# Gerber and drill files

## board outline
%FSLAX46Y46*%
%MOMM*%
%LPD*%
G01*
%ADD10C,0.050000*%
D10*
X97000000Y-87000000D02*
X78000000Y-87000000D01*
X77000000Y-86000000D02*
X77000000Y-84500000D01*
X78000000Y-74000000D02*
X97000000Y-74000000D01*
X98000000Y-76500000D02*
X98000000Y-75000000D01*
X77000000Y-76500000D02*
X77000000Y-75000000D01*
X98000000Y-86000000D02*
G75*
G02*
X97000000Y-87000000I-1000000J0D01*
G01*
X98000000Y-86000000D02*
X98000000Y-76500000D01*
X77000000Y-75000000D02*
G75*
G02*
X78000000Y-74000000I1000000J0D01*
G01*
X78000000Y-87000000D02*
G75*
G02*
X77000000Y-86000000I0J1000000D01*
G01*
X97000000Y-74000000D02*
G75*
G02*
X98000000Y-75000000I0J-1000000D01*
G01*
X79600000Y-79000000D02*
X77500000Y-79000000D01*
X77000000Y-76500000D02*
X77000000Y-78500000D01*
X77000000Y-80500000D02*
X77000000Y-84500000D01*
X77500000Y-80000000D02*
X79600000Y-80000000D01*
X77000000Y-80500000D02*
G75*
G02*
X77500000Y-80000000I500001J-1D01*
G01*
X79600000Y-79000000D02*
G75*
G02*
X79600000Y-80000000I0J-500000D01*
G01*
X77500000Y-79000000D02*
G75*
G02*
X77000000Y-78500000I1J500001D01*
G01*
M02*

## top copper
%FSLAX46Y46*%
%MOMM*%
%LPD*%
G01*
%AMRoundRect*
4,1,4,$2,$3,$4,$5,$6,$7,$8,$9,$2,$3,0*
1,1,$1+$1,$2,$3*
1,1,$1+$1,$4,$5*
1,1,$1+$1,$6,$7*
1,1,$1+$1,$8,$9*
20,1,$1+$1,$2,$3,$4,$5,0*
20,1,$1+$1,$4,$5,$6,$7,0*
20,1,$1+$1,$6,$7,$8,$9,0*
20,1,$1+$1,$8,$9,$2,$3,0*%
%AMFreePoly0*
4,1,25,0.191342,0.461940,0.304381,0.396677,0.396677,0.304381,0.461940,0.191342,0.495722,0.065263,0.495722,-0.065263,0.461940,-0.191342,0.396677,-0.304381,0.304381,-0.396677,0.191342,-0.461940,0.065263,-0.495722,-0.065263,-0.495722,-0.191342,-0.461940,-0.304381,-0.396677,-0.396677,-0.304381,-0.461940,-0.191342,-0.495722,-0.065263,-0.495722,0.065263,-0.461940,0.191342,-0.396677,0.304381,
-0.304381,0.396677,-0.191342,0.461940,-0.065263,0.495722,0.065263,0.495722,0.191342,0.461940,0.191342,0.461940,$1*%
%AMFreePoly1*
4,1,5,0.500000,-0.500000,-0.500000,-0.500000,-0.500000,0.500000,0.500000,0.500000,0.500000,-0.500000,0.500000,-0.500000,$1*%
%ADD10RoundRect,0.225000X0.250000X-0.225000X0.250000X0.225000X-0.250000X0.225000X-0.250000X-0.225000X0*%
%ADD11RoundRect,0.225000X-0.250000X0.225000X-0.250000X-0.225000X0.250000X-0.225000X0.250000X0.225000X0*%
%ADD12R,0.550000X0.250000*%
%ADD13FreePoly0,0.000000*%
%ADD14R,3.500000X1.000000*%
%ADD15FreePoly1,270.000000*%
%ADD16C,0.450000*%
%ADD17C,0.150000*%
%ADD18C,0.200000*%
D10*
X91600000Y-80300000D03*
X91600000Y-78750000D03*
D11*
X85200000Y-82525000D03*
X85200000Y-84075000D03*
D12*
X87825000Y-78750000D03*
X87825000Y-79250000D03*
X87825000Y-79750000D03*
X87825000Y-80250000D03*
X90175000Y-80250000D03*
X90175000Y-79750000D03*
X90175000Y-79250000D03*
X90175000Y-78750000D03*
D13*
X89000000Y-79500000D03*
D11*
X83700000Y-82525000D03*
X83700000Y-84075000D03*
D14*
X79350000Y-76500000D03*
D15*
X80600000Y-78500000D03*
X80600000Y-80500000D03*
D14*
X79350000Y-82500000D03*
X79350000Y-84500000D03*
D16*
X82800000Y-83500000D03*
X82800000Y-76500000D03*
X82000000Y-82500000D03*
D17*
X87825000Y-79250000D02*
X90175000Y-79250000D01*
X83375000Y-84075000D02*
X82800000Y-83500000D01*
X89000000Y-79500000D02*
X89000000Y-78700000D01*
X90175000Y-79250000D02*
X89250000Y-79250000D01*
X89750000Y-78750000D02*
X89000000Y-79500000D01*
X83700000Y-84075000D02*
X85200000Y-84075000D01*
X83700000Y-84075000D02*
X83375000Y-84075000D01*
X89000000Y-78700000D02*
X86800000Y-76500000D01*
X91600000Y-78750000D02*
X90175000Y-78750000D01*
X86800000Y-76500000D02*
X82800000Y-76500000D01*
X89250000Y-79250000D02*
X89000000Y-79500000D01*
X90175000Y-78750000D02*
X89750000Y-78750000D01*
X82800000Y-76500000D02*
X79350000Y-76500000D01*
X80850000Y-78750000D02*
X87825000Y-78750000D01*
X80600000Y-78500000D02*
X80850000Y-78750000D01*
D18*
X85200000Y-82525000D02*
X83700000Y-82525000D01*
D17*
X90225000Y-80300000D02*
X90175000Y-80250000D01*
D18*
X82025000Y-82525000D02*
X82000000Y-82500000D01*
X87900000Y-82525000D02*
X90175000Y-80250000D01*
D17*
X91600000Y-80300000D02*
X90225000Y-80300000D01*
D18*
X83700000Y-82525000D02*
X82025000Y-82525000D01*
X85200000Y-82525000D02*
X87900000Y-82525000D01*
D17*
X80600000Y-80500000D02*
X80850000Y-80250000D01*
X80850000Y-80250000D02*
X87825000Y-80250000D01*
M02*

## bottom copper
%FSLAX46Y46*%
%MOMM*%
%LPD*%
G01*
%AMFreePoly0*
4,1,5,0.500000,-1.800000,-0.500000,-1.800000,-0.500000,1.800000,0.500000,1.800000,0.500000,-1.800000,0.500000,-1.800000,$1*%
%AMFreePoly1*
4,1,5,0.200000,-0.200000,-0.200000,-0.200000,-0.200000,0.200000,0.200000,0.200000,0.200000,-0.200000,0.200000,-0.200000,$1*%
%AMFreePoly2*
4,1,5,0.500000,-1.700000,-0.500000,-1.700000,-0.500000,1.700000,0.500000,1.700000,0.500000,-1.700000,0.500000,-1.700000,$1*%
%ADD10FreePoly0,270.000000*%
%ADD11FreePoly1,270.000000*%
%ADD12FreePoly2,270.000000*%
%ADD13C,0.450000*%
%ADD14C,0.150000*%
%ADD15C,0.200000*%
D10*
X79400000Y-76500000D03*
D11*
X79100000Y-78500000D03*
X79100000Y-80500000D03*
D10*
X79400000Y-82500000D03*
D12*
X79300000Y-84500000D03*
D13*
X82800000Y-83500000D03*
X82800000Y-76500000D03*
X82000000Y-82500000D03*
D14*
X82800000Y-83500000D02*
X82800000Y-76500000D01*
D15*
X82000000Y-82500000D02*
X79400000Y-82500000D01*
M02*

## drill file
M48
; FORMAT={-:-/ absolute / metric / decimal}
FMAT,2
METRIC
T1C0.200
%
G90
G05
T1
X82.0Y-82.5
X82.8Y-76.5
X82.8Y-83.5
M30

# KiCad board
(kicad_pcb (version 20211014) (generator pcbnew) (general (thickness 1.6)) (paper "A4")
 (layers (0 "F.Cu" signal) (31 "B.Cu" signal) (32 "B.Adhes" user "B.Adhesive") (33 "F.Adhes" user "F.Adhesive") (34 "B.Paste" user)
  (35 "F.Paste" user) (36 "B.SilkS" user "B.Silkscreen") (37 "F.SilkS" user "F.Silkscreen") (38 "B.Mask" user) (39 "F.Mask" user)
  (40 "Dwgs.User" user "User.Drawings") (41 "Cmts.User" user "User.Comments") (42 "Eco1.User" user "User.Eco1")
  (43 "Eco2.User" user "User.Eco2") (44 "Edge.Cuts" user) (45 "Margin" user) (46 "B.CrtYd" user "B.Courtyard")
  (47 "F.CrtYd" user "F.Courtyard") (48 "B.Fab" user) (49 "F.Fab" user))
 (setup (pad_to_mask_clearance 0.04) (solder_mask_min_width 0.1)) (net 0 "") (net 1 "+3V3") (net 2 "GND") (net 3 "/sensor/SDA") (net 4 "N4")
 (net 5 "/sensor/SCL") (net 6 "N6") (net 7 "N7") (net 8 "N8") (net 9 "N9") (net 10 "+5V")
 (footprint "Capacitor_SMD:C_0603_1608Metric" (layer "F.Cu") (at 91.6 79.525 90)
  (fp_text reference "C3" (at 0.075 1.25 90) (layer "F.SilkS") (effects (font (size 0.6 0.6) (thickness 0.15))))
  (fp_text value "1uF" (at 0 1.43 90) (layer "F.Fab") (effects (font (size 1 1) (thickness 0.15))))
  (pad "1" smd roundrect locked (at -0.775 0 90) (size 0.9 0.95) (layers "F.Cu" "F.Paste" "F.Mask") (roundrect_rratio 0.25) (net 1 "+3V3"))
  (pad "2" smd roundrect locked (at 0.775 0 90) (size 0.9 0.95) (layers "F.Cu" "F.Paste" "F.Mask") (roundrect_rratio 0.25) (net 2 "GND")))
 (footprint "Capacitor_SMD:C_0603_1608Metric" (layer "F.Cu") (at 85.2 83.3 -90)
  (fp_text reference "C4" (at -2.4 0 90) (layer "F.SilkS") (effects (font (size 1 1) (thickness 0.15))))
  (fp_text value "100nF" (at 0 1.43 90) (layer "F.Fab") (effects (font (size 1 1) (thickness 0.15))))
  (pad "1" smd roundrect locked (at -0.775 0 270) (size 0.9 0.95) (layers "F.Cu" "F.Paste" "F.Mask") (roundrect_rratio 0.25) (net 1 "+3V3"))
  (pad "2" smd roundrect locked (at 0.775 0 270) (size 0.9 0.95) (layers "F.Cu" "F.Paste" "F.Mask") (roundrect_rratio 0.25) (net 2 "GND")))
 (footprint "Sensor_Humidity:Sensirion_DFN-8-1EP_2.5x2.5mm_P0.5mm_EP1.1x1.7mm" (layer "F.Cu") (at 89 79.5)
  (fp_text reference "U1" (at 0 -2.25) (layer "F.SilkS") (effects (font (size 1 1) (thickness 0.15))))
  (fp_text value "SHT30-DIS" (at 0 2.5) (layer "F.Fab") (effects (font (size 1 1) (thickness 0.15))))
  (pad "" smd custom (at 0 0) (size 0.9 0.9) (layers "F.Paste") (zone_connect 0) (options (clearance outline) (anchor rect)) (primitives))
  (pad "1" smd rect (at -1.175 -0.75) (size 0.55 0.25) (layers "F.Cu" "F.Paste" "F.Mask") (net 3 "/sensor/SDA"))
  (pad "2" smd rect (at -1.175 -0.25) (size 0.55 0.25) (layers "F.Cu" "F.Paste" "F.Mask") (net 2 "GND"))
  (pad "3" smd rect (at -1.175 0.25) (size 0.55 0.25) (layers "F.Cu" "F.Paste" "F.Mask") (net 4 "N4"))
  (pad "4" smd rect (at -1.175 0.75 180) (size 0.55 0.25) (layers "F.Cu" "F.Paste" "F.Mask") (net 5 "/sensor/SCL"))
  (pad "5" smd rect (at 1.175 0.75) (size 0.55 0.25) (layers "F.Cu" "F.Paste" "F.Mask") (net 1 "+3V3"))
  (pad "6" smd rect (at 1.175 0.25) (size 0.55 0.25) (layers "F.Cu" "F.Paste" "F.Mask") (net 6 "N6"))
  (pad "7" smd rect (at 1.175 -0.25) (size 0.55 0.25) (layers "F.Cu" "F.Paste" "F.Mask") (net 2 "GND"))
  (pad "8" smd rect (at 1.175 -0.75) (size 0.55 0.25) (layers "F.Cu" "F.Paste" "F.Mask") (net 2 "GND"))
  (pad "9" smd custom (at 0 0) (size 1 1) (layers "F.Cu" "F.Mask") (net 2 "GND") (zone_connect 0)
   (options (clearance outline) (anchor circle)) (primitives)))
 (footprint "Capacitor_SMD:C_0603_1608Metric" (layer "F.Cu") (at 83.7 83.3 -90)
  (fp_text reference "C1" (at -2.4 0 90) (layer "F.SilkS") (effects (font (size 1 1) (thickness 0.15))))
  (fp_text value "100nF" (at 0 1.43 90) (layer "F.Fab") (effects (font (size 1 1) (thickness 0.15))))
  (pad "1" smd roundrect (at -0.775 0 270) (size 0.9 0.95) (layers "F.Cu" "F.Paste" "F.Mask") (roundrect_rratio 0.25) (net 1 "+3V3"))
  (pad "2" smd roundrect (at 0.775 0 270) (size 0.9 0.95) (layers "F.Cu" "F.Paste" "F.Mask") (roundrect_rratio 0.25) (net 2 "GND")))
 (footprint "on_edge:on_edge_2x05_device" (layer "F.Cu") (at 77 80.5 -90)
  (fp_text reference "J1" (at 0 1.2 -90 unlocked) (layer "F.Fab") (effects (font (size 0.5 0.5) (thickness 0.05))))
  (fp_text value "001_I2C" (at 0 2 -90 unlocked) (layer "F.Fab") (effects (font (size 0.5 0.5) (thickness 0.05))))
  (fp_line (start -1.5 -2.6) (end -1.5 -0.5) (layer "Edge.Cuts") (width 0.05))
  (fp_line (start -4 0) (end -2 0) (layer "Edge.Cuts") (width 0.05))
  (fp_line (start 0 0) (end 4 0) (layer "Edge.Cuts") (width 0.05))
  (fp_line (start -0.5 -0.5) (end -0.5 -2.6) (layer "Edge.Cuts") (width 0.05))
  (fp_arc (start 0 0) (mid -0.353553 -0.146447) (end -0.5 -0.5) (layer "Edge.Cuts") (width 0.05))
  (fp_arc (start -1.5 -2.6) (mid -1 -3.1) (end -0.5 -2.6) (layer "Edge.Cuts") (width 0.05))
  (fp_arc (start -1.5 -0.5) (mid -1.646447 -0.146447) (end -2 0) (layer "Edge.Cuts") (width 0.05))
  (pad "1" smd rect locked (at -4 -2.35 90) (size 1 3.5) (layers "F.Cu" "F.Mask") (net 2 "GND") (zone_connect 0))
  (pad "2" smd custom locked (at -2 -3.6 270) (size 1 1) (layers "F.Cu" "F.Mask") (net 3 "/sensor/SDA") (zone_connect 0)
   (options (clearance outline) (anchor rect)) (primitives))
  (pad "3" smd custom locked (at 0 -3.6 270) (size 1 1) (layers "F.Cu" "F.Mask") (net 5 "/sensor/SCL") (zone_connect 0)
   (options (clearance outline) (anchor rect)) (primitives))
  (pad "4" smd rect locked (at 2 -2.35 90) (size 1 3.5) (layers "F.Cu" "F.Mask") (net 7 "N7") (zone_connect 0))
  (pad "5" smd rect locked (at 4 -2.35 90) (size 1 3.5) (layers "F.Cu" "F.Mask") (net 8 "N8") (zone_connect 0))
  (pad "6" smd custom locked (at -4 -2.4 270) (size 1 3.6) (layers "B.Cu" "B.Mask") (zone_connect 0)
   (options (clearance outline) (anchor rect)) (primitives))
  (pad "7" smd custom locked (at -2 -2.1 270) (size 0.4 0.4) (layers "B.Cu" "B.Mask") (zone_connect 0)
   (options (clearance outline) (anchor rect)) (primitives))
  (pad "8" smd custom locked (at 0 -2.1 270) (size 0.4 0.4) (layers "B.Cu" "B.Mask") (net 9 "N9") (zone_connect 0)
   (options (clearance outline) (anchor rect)) (primitives))
  (pad "9" smd custom locked (at 2 -2.4 270) (size 1 3.6) (layers "B.Cu" "B.Mask") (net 1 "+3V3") (zone_connect 0)
   (options (clearance outline) (anchor rect)) (primitives))
  (pad "10" smd custom locked (at 4 -2.3 270) (size 1 3.4) (layers "B.Cu" "B.Mask") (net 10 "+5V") (zone_connect 0)
   (options (clearance outline) (anchor rect)) (primitives)))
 (gr_line (start 97 87) (end 78 87) (layer "Edge.Cuts") (width 0.05))
 (gr_line (start 77 86) (end 77 84.5) (layer "Edge.Cuts") (width 0.05))
 (gr_line (start 78 74) (end 97 74) (layer "Edge.Cuts") (width 0.05))
 (gr_line (start 98 76.5) (end 98 75) (layer "Edge.Cuts") (width 0.05))
 (gr_line (start 77 76.5) (end 77 75) (layer "Edge.Cuts") (width 0.05))
 (gr_arc (start 98 86) (mid 97.707107 86.707107) (end 97 87) (layer "Edge.Cuts") (width 0.05))
 (gr_line (start 98 86) (end 98 76.5) (layer "Edge.Cuts") (width 0.05))
 (gr_arc (start 77 75) (mid 77.292893 74.292893) (end 78 74) (layer "Edge.Cuts") (width 0.05))
 (gr_arc (start 78 87) (mid 77.292893 86.707107) (end 77 86) (layer "Edge.Cuts") (width 0.05))
 (gr_arc (start 97 74) (mid 97.707107 74.292893) (end 98 75) (layer "Edge.Cuts") (width 0.05))
 (segment (start 87.825 79.25) (end 90.175 79.25) (width 0.15) (layer "F.Cu") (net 2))
 (segment (start 83.375 84.075) (end 82.8 83.5) (width 0.15) (layer "F.Cu") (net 2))
 (segment (start 89 79.5) (end 89 78.7) (width 0.15) (layer "F.Cu") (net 2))
 (segment (start 90.175 79.25) (end 89.25 79.25) (width 0.15) (layer "F.Cu") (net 2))
 (segment (start 89.75 78.75) (end 89 79.5) (width 0.15) (layer "F.Cu") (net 2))
 (segment (start 83.7 84.075) (end 85.2 84.075) (width 0.15) (layer "F.Cu") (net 2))
 (segment (start 83.7 84.075) (end 83.375 84.075) (width 0.15) (layer "F.Cu") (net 2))
 (segment (start 89 78.7) (end 86.8 76.5) (width 0.15) (layer "F.Cu") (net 2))
 (segment (start 91.6 78.75) (end 90.175 78.75) (width 0.15) (layer "F.Cu") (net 2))
 (segment (start 86.8 76.5) (end 82.8 76.5) (width 0.15) (layer "F.Cu") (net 2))
 (segment (start 89.25 79.25) (end 89 79.5) (width 0.15) (layer "F.Cu") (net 2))
 (segment (start 90.175 78.75) (end 89.75 78.75) (width 0.15) (layer "F.Cu") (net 2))
 (segment (start 82.8 76.5) (end 79.35 76.5) (width 0.15) (layer "F.Cu") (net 2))
 (via (at 82.8 83.5) (size 0.45) (drill 0.2) (layers "F.Cu" "B.Cu") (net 2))
 (via (at 82.8 76.5) (size 0.45) (drill 0.2) (layers "F.Cu" "B.Cu") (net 2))
 (segment (start 82.8 83.5) (end 82.8 76.5) (width 0.15) (layer "B.Cu") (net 2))
 (segment (start 80.85 78.75) (end 87.825 78.75) (width 0.15) (layer "F.Cu") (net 3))
 (segment (start 80.6 78.5) (end 80.85 78.75) (width 0.15) (layer "F.Cu") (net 3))
 (segment (start 85.2 82.525) (end 83.7 82.525) (width 0.2) (layer "F.Cu") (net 1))
 (segment (start 90.225 80.3) (end 90.175 80.25) (width 0.15) (layer "F.Cu") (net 1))
 (segment (start 82.025 82.525) (end 82 82.5) (width 0.2) (layer "F.Cu") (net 1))
 (segment (start 87.9 82.525) (end 90.175 80.25) (width 0.2) (layer "F.Cu") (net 1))
 (segment (start 91.6 80.3) (end 90.225 80.3) (width 0.15) (layer "F.Cu") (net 1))
 (segment (start 83.7 82.525) (end 82.025 82.525) (width 0.2) (layer "F.Cu") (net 1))
 (segment (start 85.2 82.525) (end 87.9 82.525) (width 0.2) (layer "F.Cu") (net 1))
 (via (at 82 82.5) (size 0.45) (drill 0.2) (layers "F.Cu" "B.Cu") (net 1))
 (segment (start 82 82.5) (end 79.4 82.5) (width 0.2) (layer "B.Cu") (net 1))
 (segment (start 80.6 80.5) (end 80.85 80.25) (width 0.15) (layer "F.Cu") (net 5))
 (segment (start 80.85 80.25) (end 87.825 80.25) (width 0.15) (layer "F.Cu") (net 5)))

